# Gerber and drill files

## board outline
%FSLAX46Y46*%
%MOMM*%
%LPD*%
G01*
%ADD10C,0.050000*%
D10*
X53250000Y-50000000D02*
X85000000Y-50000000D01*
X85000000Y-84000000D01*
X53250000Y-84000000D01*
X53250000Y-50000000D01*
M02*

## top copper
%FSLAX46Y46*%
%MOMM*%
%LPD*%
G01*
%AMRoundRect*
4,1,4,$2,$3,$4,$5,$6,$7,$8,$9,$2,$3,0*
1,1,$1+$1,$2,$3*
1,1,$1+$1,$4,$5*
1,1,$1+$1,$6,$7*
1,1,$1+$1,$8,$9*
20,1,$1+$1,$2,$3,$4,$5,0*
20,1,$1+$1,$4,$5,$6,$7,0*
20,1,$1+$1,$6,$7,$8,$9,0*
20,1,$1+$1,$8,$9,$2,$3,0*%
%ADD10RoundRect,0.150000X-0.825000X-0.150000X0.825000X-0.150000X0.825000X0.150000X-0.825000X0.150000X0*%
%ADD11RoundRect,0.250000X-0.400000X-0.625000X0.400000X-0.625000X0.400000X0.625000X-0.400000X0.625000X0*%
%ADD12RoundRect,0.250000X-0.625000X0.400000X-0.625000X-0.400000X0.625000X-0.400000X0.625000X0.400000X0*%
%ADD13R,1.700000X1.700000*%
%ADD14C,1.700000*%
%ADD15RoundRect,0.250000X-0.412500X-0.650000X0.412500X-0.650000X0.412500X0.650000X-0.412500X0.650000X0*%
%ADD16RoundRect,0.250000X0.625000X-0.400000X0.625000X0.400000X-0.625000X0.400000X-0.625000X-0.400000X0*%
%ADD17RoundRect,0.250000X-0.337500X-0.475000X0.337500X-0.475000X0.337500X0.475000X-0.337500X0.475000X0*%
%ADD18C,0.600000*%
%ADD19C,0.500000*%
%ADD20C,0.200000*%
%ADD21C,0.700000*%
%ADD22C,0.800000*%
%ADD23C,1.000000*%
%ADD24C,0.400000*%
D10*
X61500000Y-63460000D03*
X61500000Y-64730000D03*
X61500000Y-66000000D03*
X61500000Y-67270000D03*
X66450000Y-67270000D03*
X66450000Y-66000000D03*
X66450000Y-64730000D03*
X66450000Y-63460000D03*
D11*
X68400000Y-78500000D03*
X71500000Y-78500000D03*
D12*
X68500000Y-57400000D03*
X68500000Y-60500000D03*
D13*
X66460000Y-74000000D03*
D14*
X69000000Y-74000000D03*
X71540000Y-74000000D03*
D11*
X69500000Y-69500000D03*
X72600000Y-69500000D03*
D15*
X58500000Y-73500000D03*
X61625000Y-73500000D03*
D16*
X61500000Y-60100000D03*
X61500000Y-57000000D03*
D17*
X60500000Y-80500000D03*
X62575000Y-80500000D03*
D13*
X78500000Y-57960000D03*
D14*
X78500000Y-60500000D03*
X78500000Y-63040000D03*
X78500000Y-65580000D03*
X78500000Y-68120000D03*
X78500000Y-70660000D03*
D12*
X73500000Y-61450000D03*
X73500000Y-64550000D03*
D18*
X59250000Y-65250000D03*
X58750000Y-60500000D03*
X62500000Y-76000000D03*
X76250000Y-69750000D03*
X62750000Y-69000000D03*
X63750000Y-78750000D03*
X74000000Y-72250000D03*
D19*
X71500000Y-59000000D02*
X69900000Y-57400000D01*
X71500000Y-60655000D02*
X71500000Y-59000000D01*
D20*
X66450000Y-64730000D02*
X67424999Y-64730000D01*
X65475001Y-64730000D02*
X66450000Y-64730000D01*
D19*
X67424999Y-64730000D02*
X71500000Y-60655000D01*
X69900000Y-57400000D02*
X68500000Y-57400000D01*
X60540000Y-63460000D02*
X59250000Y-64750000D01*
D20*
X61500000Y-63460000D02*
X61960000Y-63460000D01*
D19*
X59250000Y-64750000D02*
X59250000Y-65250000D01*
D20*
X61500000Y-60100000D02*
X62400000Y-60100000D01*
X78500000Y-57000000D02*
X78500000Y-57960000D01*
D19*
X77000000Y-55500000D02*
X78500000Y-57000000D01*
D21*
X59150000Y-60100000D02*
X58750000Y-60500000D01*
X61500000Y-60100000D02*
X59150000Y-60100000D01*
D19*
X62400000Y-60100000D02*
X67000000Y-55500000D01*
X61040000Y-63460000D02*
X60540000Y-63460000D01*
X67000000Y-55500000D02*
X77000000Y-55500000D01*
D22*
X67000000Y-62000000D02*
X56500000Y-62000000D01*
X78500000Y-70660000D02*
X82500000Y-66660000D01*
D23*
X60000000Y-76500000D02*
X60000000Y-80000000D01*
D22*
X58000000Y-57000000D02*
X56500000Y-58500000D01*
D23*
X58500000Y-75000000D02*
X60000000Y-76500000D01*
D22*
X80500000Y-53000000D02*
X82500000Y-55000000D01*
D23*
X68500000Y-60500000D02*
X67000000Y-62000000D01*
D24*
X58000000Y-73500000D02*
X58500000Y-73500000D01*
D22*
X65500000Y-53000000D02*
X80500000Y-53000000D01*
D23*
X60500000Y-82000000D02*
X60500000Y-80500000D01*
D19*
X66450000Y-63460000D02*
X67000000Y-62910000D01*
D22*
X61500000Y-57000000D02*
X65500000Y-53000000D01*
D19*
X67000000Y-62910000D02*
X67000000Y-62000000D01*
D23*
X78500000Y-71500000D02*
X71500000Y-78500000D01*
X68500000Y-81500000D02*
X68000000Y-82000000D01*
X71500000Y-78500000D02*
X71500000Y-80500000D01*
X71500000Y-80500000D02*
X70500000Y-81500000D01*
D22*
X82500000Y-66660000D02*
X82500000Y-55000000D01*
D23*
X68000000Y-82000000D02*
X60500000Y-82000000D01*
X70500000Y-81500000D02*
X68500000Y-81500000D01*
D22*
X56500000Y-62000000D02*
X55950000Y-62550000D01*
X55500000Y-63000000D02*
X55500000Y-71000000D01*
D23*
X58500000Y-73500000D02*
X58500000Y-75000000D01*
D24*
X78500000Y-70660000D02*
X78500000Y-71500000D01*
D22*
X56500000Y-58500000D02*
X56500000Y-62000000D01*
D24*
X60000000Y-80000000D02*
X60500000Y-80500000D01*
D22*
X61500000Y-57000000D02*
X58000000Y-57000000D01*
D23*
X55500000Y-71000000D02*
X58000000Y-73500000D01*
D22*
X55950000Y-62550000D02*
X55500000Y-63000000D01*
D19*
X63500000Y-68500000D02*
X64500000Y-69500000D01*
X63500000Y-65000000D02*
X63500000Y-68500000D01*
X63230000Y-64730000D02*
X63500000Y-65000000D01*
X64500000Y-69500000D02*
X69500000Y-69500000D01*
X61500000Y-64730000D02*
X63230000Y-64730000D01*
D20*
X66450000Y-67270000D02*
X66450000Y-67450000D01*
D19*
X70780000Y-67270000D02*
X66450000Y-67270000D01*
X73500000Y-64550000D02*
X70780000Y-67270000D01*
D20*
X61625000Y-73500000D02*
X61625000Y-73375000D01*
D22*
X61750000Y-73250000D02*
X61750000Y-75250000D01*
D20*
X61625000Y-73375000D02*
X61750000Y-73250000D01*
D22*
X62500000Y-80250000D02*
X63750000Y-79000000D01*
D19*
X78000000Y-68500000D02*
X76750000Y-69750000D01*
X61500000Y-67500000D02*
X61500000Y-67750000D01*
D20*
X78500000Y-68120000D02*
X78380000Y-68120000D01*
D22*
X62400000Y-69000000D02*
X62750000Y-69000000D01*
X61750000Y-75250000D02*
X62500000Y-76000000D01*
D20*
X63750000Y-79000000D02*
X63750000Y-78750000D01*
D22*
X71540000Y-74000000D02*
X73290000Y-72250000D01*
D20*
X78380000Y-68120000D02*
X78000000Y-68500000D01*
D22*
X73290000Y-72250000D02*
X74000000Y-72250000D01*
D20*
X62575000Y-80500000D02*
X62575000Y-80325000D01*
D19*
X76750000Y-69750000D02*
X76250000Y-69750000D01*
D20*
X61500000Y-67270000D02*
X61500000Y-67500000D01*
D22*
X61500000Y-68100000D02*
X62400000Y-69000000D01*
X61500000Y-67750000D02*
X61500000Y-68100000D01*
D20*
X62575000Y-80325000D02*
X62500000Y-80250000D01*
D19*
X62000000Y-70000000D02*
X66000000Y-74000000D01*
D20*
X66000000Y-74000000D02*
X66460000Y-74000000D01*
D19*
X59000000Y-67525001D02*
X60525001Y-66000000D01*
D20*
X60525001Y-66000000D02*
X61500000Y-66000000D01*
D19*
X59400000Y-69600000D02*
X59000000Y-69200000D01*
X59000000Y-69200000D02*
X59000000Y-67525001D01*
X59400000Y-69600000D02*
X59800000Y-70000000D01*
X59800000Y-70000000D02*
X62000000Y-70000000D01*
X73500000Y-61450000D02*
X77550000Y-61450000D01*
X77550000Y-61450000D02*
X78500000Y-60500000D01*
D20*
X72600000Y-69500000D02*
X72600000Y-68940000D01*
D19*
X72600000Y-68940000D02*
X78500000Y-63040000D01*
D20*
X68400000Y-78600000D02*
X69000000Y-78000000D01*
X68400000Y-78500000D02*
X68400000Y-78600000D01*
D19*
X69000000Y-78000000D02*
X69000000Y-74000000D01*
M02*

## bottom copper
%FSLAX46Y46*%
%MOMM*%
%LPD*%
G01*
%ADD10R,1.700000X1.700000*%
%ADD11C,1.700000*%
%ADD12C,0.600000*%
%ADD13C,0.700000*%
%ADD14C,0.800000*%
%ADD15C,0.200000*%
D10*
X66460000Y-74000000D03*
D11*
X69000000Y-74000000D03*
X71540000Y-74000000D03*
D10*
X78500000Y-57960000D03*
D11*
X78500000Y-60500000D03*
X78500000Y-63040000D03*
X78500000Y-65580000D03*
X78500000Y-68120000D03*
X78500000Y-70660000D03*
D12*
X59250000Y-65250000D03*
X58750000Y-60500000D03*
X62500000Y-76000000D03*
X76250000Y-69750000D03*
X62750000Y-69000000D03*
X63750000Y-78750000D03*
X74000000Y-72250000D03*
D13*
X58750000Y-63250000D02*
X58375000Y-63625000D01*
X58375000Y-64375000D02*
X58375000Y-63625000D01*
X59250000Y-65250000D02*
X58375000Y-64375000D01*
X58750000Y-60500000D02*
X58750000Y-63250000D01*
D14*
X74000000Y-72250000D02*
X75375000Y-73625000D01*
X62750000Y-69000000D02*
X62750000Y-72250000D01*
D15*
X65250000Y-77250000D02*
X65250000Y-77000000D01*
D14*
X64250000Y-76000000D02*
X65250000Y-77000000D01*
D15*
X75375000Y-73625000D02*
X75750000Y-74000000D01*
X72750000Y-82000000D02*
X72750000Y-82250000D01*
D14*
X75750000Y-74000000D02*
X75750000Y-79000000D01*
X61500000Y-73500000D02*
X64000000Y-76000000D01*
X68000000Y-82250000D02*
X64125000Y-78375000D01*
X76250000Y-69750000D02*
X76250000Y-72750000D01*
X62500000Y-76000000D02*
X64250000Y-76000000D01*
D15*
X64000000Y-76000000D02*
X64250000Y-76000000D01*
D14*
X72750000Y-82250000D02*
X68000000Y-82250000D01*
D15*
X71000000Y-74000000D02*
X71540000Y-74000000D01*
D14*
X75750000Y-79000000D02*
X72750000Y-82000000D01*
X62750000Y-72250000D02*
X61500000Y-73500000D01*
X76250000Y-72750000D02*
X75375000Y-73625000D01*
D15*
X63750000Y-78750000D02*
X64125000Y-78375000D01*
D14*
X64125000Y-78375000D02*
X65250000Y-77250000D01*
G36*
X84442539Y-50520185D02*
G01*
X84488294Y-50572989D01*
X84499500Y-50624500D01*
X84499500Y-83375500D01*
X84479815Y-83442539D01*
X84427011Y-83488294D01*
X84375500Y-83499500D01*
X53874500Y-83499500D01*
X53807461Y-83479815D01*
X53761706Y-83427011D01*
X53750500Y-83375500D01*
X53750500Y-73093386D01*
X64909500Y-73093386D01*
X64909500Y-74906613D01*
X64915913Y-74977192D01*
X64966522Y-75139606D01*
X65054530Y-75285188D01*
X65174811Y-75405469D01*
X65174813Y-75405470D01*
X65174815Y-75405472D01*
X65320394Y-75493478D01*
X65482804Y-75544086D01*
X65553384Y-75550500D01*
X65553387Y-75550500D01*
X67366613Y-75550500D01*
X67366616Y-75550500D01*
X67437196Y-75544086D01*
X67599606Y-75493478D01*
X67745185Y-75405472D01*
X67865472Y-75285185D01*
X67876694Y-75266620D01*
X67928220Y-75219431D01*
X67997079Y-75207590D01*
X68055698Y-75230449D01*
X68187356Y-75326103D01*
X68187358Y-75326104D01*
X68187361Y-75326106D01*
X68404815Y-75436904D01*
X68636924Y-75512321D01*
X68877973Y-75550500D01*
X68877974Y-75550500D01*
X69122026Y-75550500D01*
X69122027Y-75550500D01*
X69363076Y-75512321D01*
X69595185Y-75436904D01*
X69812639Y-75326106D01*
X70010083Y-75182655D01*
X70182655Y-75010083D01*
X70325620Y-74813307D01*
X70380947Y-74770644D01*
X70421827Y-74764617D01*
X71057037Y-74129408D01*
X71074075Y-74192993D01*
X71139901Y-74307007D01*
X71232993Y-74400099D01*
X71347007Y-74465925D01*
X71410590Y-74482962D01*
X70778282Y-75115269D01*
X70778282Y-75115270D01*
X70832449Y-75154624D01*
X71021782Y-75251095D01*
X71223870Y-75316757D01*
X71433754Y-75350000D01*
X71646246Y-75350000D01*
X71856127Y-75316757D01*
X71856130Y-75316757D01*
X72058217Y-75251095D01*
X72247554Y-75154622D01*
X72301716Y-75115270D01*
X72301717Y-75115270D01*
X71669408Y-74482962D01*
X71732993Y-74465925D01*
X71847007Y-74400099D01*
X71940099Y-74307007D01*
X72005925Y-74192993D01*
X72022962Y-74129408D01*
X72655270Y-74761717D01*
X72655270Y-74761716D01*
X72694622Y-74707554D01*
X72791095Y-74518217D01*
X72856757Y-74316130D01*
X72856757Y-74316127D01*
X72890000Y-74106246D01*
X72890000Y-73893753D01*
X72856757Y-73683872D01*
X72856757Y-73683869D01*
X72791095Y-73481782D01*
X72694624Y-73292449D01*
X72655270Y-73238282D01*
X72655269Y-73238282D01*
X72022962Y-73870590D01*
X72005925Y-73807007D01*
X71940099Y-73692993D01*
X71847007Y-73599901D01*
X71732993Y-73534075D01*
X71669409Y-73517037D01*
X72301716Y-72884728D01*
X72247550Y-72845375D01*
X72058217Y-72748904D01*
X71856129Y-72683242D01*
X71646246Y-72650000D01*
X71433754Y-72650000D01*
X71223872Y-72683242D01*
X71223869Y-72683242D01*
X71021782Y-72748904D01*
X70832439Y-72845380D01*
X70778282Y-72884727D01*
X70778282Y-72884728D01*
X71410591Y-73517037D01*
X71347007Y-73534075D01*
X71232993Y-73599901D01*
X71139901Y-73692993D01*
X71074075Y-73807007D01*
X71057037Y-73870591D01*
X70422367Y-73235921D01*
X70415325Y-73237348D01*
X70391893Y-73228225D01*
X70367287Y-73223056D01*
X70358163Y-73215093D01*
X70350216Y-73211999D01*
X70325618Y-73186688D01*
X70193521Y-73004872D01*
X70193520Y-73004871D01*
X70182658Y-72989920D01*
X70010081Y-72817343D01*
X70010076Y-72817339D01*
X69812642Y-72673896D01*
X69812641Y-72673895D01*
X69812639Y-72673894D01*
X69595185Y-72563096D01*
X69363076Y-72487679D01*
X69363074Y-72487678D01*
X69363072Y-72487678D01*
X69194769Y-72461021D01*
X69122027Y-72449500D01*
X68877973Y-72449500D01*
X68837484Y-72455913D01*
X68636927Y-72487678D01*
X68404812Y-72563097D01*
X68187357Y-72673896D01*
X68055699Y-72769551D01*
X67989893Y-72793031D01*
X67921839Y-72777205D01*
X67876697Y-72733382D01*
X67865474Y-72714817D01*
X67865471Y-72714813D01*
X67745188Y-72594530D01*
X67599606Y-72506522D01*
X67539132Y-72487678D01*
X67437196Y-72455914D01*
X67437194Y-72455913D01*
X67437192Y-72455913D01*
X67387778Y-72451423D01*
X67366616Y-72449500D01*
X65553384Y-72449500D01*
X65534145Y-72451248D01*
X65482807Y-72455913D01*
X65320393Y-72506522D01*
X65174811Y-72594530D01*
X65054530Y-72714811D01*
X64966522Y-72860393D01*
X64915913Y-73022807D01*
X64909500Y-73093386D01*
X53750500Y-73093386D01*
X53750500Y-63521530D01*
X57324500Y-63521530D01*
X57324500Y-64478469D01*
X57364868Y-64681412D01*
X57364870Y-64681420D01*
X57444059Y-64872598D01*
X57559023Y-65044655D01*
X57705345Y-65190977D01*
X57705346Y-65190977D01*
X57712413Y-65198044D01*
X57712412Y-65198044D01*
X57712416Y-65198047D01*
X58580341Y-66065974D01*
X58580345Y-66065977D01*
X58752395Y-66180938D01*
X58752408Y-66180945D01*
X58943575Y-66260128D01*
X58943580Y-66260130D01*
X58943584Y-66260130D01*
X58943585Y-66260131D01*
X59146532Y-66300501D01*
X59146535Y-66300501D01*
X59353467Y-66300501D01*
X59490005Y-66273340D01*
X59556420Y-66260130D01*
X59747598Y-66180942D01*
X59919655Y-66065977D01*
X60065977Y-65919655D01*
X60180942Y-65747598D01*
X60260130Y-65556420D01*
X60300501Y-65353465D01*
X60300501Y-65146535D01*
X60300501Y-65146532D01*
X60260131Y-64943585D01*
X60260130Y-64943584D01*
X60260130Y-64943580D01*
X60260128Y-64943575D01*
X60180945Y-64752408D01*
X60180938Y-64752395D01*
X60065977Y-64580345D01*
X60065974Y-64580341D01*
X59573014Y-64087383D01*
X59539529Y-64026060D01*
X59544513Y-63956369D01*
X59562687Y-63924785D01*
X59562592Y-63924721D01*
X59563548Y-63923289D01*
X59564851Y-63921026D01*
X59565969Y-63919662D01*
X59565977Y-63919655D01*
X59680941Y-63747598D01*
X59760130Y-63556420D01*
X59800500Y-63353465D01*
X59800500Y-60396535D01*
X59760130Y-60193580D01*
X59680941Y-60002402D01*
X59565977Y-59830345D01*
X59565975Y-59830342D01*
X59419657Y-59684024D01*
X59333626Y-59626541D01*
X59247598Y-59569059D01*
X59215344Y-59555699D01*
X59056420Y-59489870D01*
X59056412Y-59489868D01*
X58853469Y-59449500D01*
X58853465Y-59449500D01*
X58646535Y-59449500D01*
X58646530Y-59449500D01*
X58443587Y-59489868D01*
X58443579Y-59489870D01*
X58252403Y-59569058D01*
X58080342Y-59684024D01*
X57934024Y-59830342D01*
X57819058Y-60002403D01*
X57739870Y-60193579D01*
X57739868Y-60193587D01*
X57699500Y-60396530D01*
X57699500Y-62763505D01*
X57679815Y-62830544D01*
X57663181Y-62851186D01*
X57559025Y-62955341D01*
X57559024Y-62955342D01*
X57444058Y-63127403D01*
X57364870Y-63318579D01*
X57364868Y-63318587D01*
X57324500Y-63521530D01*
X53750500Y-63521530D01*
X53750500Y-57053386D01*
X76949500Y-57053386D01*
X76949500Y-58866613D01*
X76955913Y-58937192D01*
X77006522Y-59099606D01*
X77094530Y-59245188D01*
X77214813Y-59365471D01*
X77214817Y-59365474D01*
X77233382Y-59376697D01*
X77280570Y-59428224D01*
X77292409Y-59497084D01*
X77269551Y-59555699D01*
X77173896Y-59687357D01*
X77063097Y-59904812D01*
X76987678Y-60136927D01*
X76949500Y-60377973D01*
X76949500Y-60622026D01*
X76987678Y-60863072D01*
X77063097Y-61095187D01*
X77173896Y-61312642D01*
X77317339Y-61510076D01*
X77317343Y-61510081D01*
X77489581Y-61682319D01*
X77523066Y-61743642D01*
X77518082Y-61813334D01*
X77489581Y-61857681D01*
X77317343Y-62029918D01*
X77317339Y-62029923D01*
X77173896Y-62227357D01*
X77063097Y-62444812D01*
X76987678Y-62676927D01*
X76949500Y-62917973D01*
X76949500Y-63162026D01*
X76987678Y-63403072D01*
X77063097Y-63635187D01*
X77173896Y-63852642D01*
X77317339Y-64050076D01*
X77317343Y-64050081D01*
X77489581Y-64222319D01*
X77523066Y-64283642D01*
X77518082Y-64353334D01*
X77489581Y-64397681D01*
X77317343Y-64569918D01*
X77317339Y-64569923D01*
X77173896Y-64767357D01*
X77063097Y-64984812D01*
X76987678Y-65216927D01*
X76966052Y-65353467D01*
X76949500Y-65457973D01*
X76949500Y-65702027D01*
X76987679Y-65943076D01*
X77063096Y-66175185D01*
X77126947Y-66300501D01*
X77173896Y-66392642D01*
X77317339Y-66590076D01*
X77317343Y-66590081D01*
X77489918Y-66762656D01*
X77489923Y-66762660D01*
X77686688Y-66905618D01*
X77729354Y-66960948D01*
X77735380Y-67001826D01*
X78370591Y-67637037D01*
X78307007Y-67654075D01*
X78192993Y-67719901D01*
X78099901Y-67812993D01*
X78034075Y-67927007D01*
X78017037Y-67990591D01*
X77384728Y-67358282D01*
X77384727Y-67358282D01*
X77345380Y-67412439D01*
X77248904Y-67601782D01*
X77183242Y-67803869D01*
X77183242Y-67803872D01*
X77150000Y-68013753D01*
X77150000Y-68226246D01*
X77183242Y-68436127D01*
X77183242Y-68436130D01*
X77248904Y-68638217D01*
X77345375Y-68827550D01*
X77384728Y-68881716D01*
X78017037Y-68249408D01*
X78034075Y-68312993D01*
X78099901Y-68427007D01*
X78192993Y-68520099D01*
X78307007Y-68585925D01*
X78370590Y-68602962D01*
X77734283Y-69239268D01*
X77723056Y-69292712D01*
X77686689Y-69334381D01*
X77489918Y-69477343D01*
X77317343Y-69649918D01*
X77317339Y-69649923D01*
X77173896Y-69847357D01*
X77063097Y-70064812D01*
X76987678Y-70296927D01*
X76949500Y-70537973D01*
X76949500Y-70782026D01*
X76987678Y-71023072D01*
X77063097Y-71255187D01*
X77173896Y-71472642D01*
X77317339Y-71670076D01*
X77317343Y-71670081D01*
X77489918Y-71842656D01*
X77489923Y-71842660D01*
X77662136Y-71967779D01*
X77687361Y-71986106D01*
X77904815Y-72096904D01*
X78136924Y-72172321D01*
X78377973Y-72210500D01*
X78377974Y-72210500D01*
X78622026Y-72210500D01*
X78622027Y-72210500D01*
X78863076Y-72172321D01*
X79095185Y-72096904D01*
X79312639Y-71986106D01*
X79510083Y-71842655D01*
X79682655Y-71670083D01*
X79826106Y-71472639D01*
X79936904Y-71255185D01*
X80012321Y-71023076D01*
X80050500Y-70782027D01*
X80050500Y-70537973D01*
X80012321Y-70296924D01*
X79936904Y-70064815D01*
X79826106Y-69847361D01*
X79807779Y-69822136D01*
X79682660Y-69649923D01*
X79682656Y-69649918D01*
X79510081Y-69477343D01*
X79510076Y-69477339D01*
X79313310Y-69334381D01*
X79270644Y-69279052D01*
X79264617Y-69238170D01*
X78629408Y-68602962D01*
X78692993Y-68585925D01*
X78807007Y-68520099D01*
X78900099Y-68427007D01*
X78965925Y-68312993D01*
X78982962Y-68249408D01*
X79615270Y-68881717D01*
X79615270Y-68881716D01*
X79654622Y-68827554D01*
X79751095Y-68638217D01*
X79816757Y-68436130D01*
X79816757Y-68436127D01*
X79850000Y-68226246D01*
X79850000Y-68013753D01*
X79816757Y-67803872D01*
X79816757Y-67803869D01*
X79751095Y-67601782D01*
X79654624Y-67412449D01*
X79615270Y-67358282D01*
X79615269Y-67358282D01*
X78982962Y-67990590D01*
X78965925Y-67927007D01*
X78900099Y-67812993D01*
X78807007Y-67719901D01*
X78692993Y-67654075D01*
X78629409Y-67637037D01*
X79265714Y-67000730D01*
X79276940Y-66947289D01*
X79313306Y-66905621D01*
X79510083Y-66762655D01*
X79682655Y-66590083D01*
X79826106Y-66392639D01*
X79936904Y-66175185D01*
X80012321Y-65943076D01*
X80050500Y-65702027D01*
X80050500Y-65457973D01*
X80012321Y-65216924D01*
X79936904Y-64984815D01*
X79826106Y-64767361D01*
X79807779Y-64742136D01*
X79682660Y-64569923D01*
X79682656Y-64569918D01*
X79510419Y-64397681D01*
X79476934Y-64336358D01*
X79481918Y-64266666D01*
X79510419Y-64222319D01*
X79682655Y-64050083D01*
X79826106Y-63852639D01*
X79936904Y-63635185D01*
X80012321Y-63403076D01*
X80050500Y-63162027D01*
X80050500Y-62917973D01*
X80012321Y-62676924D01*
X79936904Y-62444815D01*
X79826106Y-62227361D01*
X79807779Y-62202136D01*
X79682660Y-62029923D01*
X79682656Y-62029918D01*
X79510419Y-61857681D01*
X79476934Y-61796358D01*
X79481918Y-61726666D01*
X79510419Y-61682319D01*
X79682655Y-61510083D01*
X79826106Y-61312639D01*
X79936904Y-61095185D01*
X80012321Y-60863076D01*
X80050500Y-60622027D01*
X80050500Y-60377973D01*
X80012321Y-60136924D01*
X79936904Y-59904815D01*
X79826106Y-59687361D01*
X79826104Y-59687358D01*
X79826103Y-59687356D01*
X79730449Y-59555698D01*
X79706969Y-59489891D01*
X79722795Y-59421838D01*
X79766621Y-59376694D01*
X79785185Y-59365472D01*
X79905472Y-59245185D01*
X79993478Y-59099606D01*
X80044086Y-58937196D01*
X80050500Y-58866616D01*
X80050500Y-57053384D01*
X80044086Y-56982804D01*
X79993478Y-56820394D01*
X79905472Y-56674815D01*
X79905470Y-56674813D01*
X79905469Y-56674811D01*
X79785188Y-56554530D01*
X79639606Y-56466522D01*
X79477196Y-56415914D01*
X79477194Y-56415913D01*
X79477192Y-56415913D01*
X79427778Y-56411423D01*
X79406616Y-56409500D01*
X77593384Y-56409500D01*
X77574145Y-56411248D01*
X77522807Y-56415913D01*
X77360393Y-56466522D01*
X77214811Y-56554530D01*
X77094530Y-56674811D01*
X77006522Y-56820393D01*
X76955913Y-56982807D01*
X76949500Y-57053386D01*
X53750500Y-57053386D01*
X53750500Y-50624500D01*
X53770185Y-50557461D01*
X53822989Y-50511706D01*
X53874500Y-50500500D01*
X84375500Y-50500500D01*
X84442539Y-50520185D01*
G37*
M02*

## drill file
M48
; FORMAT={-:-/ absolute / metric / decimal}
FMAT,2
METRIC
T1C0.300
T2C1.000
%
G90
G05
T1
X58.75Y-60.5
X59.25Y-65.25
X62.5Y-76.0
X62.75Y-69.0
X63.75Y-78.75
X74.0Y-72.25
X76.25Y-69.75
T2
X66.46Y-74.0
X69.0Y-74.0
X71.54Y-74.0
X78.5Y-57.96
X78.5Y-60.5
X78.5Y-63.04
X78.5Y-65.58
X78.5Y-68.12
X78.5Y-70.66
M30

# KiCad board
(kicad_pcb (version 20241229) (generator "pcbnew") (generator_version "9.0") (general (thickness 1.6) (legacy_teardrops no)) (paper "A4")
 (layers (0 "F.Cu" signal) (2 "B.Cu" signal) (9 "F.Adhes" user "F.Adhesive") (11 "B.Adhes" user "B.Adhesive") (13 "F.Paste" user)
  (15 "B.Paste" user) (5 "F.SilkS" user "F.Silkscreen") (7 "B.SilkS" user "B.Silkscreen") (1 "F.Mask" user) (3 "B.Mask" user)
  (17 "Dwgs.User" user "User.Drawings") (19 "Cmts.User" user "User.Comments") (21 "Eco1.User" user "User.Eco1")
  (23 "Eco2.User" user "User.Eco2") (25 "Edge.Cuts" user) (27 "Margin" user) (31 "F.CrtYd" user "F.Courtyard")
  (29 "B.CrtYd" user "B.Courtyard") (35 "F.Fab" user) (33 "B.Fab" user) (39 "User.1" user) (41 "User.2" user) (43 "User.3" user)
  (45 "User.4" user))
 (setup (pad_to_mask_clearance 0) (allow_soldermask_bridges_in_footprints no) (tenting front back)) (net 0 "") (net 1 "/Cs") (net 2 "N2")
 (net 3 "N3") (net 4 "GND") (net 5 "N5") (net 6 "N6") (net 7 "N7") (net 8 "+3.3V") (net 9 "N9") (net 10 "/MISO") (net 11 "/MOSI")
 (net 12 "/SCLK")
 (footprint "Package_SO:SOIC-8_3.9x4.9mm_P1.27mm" (layer "F.Cu") (at 63.975 65.365)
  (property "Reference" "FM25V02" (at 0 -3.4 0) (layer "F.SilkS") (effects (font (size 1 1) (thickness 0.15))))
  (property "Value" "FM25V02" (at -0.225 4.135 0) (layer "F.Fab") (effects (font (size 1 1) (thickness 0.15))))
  (pad "1" smd roundrect (at -2.475 -1.905) (size 1.95 0.6) (layers "F.Cu" "F.Mask" "F.Paste") (roundrect_rratio 0.25) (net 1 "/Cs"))
  (pad "2" smd roundrect (at -2.475 -0.635) (size 1.95 0.6) (layers "F.Cu" "F.Mask" "F.Paste") (roundrect_rratio 0.25) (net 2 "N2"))
  (pad "3" smd roundrect (at -2.475 0.635) (size 1.95 0.6) (layers "F.Cu" "F.Mask" "F.Paste") (roundrect_rratio 0.25) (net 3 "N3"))
  (pad "4" smd roundrect (at -2.475 1.905) (size 1.95 0.6) (layers "F.Cu" "F.Mask" "F.Paste") (roundrect_rratio 0.25) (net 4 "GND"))
  (pad "5" smd roundrect (at 2.475 1.905) (size 1.95 0.6) (layers "F.Cu" "F.Mask" "F.Paste") (roundrect_rratio 0.25) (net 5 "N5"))
  (pad "6" smd roundrect (at 2.475 0.635) (size 1.95 0.6) (layers "F.Cu" "F.Mask" "F.Paste") (roundrect_rratio 0.25) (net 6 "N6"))
  (pad "7" smd roundrect (at 2.475 -0.635) (size 1.95 0.6) (layers "F.Cu" "F.Mask" "F.Paste") (roundrect_rratio 0.25) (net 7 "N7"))
  (pad "8" smd roundrect (at 2.475 -1.905) (size 1.95 0.6) (layers "F.Cu" "F.Mask" "F.Paste") (roundrect_rratio 0.25) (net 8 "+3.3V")))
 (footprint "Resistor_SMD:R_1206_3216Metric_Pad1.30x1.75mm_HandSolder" (layer "F.Cu") (at 69.95 78.5)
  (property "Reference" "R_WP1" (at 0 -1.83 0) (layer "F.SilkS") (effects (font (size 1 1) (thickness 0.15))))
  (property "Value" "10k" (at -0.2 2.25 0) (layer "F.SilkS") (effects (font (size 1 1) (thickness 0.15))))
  (pad "1" smd roundrect (at -1.55 0) (size 1.3 1.75) (layers "F.Cu" "F.Mask" "F.Paste") (roundrect_rratio 0.192308) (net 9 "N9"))
  (pad "2" smd roundrect (at 1.55 0) (size 1.3 1.75) (layers "F.Cu" "F.Mask" "F.Paste") (roundrect_rratio 0.192308) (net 8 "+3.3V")))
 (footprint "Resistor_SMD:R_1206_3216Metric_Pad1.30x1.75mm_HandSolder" (layer "F.Cu") (at 68.5 58.95 -90)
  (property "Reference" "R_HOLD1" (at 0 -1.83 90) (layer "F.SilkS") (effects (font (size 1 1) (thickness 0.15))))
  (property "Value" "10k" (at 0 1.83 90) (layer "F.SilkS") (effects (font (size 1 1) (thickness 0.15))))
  (pad "1" smd roundrect (at -1.55 0 270) (size 1.3 1.75) (layers "F.Cu" "F.Mask" "F.Paste") (roundrect_rratio 0.192308) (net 7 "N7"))
  (pad "2" smd roundrect (at 1.55 0 270) (size 1.3 1.75) (layers "F.Cu" "F.Mask" "F.Paste") (roundrect_rratio 0.192308) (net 8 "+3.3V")))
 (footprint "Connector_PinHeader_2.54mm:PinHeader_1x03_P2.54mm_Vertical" (layer "F.Cu") (at 66.46 74 90)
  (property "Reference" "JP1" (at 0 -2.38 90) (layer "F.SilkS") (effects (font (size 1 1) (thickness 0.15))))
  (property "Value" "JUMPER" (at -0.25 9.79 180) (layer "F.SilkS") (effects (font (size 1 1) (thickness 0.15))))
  (pad "1" thru_hole rect (at 0 0 90) (size 1.7 1.7) (drill 1) (layers "*.Cu" "*.Mask") (remove_unused_layers no) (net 3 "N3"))
  (pad "2" thru_hole circle (at 0 2.54 90) (size 1.7 1.7) (drill 1) (layers "*.Cu" "*.Mask") (remove_unused_layers no) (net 9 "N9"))
  (pad "3" thru_hole circle (at 0 5.08 90) (size 1.7 1.7) (drill 1) (layers "*.Cu" "*.Mask") (remove_unused_layers no) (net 4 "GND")))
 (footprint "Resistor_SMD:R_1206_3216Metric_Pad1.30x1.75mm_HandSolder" (layer "F.Cu") (at 71.05 69.5)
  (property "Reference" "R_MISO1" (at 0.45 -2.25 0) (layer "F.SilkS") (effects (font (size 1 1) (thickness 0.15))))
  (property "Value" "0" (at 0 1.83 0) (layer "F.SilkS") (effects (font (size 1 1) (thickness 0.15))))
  (pad "1" smd roundrect (at -1.55 0) (size 1.3 1.75) (layers "F.Cu" "F.Mask" "F.Paste") (roundrect_rratio 0.192308) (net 2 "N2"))
  (pad "2" smd roundrect (at 1.55 0) (size 1.3 1.75) (layers "F.Cu" "F.Mask" "F.Paste") (roundrect_rratio 0.192308) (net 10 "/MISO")))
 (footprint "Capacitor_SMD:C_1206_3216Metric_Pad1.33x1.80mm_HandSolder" (layer "F.Cu") (at 60.0625 73.5)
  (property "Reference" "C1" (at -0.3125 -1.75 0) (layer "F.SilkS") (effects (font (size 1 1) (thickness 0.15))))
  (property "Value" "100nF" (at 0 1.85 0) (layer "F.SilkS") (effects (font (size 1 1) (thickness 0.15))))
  (pad "1" smd roundrect (at -1.5625 0) (size 1.325 1.8) (layers "F.Cu" "F.Mask" "F.Paste") (roundrect_rratio 0.188679) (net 8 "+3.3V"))
  (pad "2" smd roundrect (at 1.5625 0) (size 1.325 1.8) (layers "F.Cu" "F.Mask" "F.Paste") (roundrect_rratio 0.188679) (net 4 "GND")))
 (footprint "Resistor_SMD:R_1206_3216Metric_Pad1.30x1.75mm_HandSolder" (layer "F.Cu") (at 61.5 58.55 90)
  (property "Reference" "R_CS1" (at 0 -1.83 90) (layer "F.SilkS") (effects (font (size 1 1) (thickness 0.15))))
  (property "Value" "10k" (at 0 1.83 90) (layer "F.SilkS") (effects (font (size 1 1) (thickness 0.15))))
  (pad "1" smd roundrect (at -1.55 0 90) (size 1.3 1.75) (layers "F.Cu" "F.Mask" "F.Paste") (roundrect_rratio 0.192308) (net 1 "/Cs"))
  (pad "2" smd roundrect (at 1.55 0 90) (size 1.3 1.75) (layers "F.Cu" "F.Mask" "F.Paste") (roundrect_rratio 0.192308) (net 8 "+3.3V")))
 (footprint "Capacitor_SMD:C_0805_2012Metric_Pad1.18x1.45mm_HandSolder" (layer "F.Cu") (at 61.5375 80.5)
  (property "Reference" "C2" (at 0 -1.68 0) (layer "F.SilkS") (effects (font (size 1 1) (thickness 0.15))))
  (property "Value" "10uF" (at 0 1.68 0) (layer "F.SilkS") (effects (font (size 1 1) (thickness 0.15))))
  (pad "1" smd roundrect (at -1.0375 0) (size 1.175 1.45) (layers "F.Cu" "F.Mask" "F.Paste") (roundrect_rratio 0.212766) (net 8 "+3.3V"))
  (pad "2" smd roundrect (at 1.0375 0) (size 1.175 1.45) (layers "F.Cu" "F.Mask" "F.Paste") (roundrect_rratio 0.212766) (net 4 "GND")))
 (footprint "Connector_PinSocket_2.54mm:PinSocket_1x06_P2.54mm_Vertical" (layer "F.Cu") (at 78.5 57.96)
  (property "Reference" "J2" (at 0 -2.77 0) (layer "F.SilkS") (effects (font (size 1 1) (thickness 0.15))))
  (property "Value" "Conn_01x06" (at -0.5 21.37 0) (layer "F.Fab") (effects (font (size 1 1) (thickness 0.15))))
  (pad "1" thru_hole rect (at 0 0) (size 1.7 1.7) (drill 1) (layers "*.Cu" "*.Mask") (remove_unused_layers no) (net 1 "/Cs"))
  (pad "2" thru_hole circle (at 0 2.54) (size 1.7 1.7) (drill 1) (layers "*.Cu" "*.Mask") (remove_unused_layers no) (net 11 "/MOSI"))
  (pad "3" thru_hole circle (at 0 5.08) (size 1.7 1.7) (drill 1) (layers "*.Cu" "*.Mask") (remove_unused_layers no) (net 10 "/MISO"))
  (pad "4" thru_hole circle (at 0 7.62) (size 1.7 1.7) (drill 1) (layers "*.Cu" "*.Mask") (remove_unused_layers no) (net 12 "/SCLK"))
  (pad "5" thru_hole circle (at 0 10.16) (size 1.7 1.7) (drill 1) (layers "*.Cu" "*.Mask") (remove_unused_layers no) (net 4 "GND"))
  (pad "6" thru_hole circle (at 0 12.7) (size 1.7 1.7) (drill 1) (layers "*.Cu" "*.Mask") (remove_unused_layers no) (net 8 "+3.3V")))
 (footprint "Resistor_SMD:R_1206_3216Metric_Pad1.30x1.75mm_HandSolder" (layer "F.Cu") (at 73.5 63 -90)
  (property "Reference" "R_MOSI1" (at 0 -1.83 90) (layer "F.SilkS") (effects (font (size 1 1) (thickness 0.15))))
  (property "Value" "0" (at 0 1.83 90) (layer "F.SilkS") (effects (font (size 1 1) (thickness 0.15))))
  (pad "1" smd roundrect (at -1.55 0 270) (size 1.3 1.75) (layers "F.Cu" "F.Mask" "F.Paste") (roundrect_rratio 0.192308) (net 11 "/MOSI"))
  (pad "2" smd roundrect (at 1.55 0 270) (size 1.3 1.75) (layers "F.Cu" "F.Mask" "F.Paste") (roundrect_rratio 0.192308) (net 5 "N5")))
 (gr_rect (start 53.25 50) (end 85 84) (stroke (width 0.05) (type default)) (fill no) (layer "Edge.Cuts"))
 (segment (start 71.5 59) (end 69.9 57.4) (width 0.5) (layer "F.Cu") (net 7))
 (segment (start 71.5 60.655) (end 71.5 59) (width 0.5) (layer "F.Cu") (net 7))
 (segment (start 66.45 64.73) (end 67.424999 64.73) (width 0.2) (layer "F.Cu") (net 7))
 (segment (start 65.475001 64.73) (end 66.45 64.73) (width 0.2) (layer "F.Cu") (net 7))
 (segment (start 67.424999 64.73) (end 71.5 60.655) (width 0.5) (layer "F.Cu") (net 7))
 (segment (start 69.9 57.4) (end 68.5 57.4) (width 0.5) (layer "F.Cu") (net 7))
 (segment (start 60.54 63.46) (end 59.25 64.75) (width 0.5) (layer "F.Cu") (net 1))
 (segment (start 61.5 63.46) (end 61.96 63.46) (width 0.2) (layer "F.Cu") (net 1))
 (segment (start 59.25 64.75) (end 59.25 65.25) (width 0.5) (layer "F.Cu") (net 1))
 (segment (start 61.5 60.1) (end 62.4 60.1) (width 0.2) (layer "F.Cu") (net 1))
 (segment (start 78.5 57) (end 78.5 57.96) (width 0.2) (layer "F.Cu") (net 1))
 (segment (start 77 55.5) (end 78.5 57) (width 0.5) (layer "F.Cu") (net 1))
 (segment (start 59.15 60.1) (end 58.75 60.5) (width 0.7) (layer "F.Cu") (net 1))
 (segment (start 61.5 60.1) (end 59.15 60.1) (width 0.7) (layer "F.Cu") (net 1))
 (segment (start 62.4 60.1) (end 67 55.5) (width 0.5) (layer "F.Cu") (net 1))
 (segment (start 61.04 63.46) (end 60.54 63.46) (width 0.5) (layer "F.Cu") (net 1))
 (segment (start 67 55.5) (end 77 55.5) (width 0.5) (layer "F.Cu") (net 1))
 (via (at 59.25 65.25) (size 0.6) (drill 0.3) (layers "F.Cu" "B.Cu") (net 1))
 (via (at 58.75 60.5) (size 0.6) (drill 0.3) (layers "F.Cu" "B.Cu") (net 1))
 (segment (start 58.75 63.25) (end 58.375 63.625) (width 0.7) (layer "B.Cu") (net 1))
 (segment (start 58.375 64.375) (end 58.375 63.625) (width 0.7) (layer "B.Cu") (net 1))
 (segment (start 59.25 65.25) (end 58.375 64.375) (width 0.7) (layer "B.Cu") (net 1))
 (segment (start 58.75 60.5) (end 58.75 63.25) (width 0.7) (layer "B.Cu") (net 1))
 (segment (start 67 62) (end 56.5 62) (width 0.8) (layer "F.Cu") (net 8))
 (segment (start 78.5 70.66) (end 82.5 66.66) (width 0.8) (layer "F.Cu") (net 8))
 (segment (start 60 76.5) (end 60 80) (width 1) (layer "F.Cu") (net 8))
 (segment (start 58 57) (end 56.5 58.5) (width 0.8) (layer "F.Cu") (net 8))
 (segment (start 58.5 75) (end 60 76.5) (width 1) (layer "F.Cu") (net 8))
 (segment (start 80.5 53) (end 82.5 55) (width 0.8) (layer "F.Cu") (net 8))
 (segment (start 68.5 60.5) (end 67 62) (width 1) (layer "F.Cu") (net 8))
 (segment (start 58 73.5) (end 58.5 73.5) (width 0.4) (layer "F.Cu") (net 8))
 (segment (start 65.5 53) (end 80.5 53) (width 0.8) (layer "F.Cu") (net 8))
 (segment (start 60.5 82) (end 60.5 80.5) (width 1) (layer "F.Cu") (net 8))
 (segment (start 66.45 63.46) (end 67 62.91) (width 0.5) (layer "F.Cu") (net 8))
 (segment (start 61.5 57) (end 65.5 53) (width 0.8) (layer "F.Cu") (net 8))
 (segment (start 67 62.91) (end 67 62) (width 0.5) (layer "F.Cu") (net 8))
 (segment (start 78.5 71.5) (end 71.5 78.5) (width 1) (layer "F.Cu") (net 8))
 (segment (start 68.5 81.5) (end 68 82) (width 1) (layer "F.Cu") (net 8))
 (segment (start 71.5 78.5) (end 71.5 80.5) (width 1) (layer "F.Cu") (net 8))
 (segment (start 71.5 80.5) (end 70.5 81.5) (width 1) (layer "F.Cu") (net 8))
 (segment (start 82.5 66.66) (end 82.5 55) (width 0.8) (layer "F.Cu") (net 8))
 (segment (start 68 82) (end 60.5 82) (width 1) (layer "F.Cu") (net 8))
 (segment (start 70.5 81.5) (end 68.5 81.5) (width 1) (layer "F.Cu") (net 8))
 (segment (start 56.5 62) (end 55.95 62.55) (width 0.8) (layer "F.Cu") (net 8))
 (segment (start 55.5 63) (end 55.5 71) (width 0.8) (layer "F.Cu") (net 8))
 (segment (start 58.5 73.5) (end 58.5 75) (width 1) (layer "F.Cu") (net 8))
 (segment (start 78.5 70.66) (end 78.5 71.5) (width 0.4) (layer "F.Cu") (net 8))
 (segment (start 56.5 58.5) (end 56.5 62) (width 0.8) (layer "F.Cu") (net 8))
 (segment (start 60 80) (end 60.5 80.5) (width 0.4) (layer "F.Cu") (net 8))
 (segment (start 61.5 57) (end 58 57) (width 0.8) (layer "F.Cu") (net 8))
 (segment (start 55.5 71) (end 58 73.5) (width 1) (layer "F.Cu") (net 8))
 (segment (start 55.95 62.55) (end 55.5 63) (width 0.8) (layer "F.Cu") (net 8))
 (segment (start 63.5 68.5) (end 64.5 69.5) (width 0.5) (layer "F.Cu") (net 2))
 (segment (start 63.5 65) (end 63.5 68.5) (width 0.5) (layer "F.Cu") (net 2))
 (segment (start 63.23 64.73) (end 63.5 65) (width 0.5) (layer "F.Cu") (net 2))
 (segment (start 64.5 69.5) (end 69.5 69.5) (width 0.5) (layer "F.Cu") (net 2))
 (segment (start 61.5 64.73) (end 63.23 64.73) (width 0.5) (layer "F.Cu") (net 2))
 (segment (start 66.45 67.27) (end 66.45 67.45) (width 0.2) (layer "F.Cu") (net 5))
 (segment (start 70.78 67.27) (end 66.45 67.27) (width 0.5) (layer "F.Cu") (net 5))
 (segment (start 73.5 64.55) (end 70.78 67.27) (width 0.5) (layer "F.Cu") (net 5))
 (segment (start 61.625 73.5) (end 61.625 73.375) (width 0.2) (layer "F.Cu") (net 4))
 (segment (start 61.75 73.25) (end 61.75 75.25) (width 0.8) (layer "F.Cu") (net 4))
 (segment (start 61.625 73.375) (end 61.75 73.25) (width 0.2) (layer "F.Cu") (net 4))
 (segment (start 62.5 80.25) (end 63.75 79) (width 0.8) (layer "F.Cu") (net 4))
 (segment (start 78 68.5) (end 76.75 69.75) (width 0.5) (layer "F.Cu") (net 4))
 (segment (start 61.5 67.5) (end 61.5 67.75) (width 0.5) (layer "F.Cu") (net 4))
 (segment (start 78.5 68.12) (end 78.38 68.12) (width 0.2) (layer "F.Cu") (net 4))
 (segment (start 62.4 69) (end 62.75 69) (width 0.8) (layer "F.Cu") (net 4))
 (segment (start 61.75 75.25) (end 62.5 76) (width 0.8) (layer "F.Cu") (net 4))
 (segment (start 63.75 79) (end 63.75 78.75) (width 0.2) (layer "F.Cu") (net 4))
 (segment (start 71.54 74) (end 73.29 72.25) (width 0.8) (layer "F.Cu") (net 4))
 (segment (start 78.38 68.12) (end 78 68.5) (width 0.2) (layer "F.Cu") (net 4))
 (segment (start 73.29 72.25) (end 74 72.25) (width 0.8) (layer "F.Cu") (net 4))
 (segment (start 62.575 80.5) (end 62.575 80.325) (width 0.2) (layer "F.Cu") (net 4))
 (segment (start 76.75 69.75) (end 76.25 69.75) (width 0.5) (layer "F.Cu") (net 4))
 (segment (start 61.5 67.27) (end 61.5 67.5) (width 0.2) (layer "F.Cu") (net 4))
 (segment (start 61.5 68.1) (end 62.4 69) (width 0.8) (layer "F.Cu") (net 4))
 (segment (start 61.5 67.75) (end 61.5 68.1) (width 0.8) (layer "F.Cu") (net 4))
 (segment (start 62.575 80.325) (end 62.5 80.25) (width 0.2) (layer "F.Cu") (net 4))
 (via (at 62.5 76) (size 0.6) (drill 0.3) (layers "F.Cu" "B.Cu") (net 4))
 (via (at 76.25 69.75) (size 0.6) (drill 0.3) (layers "F.Cu" "B.Cu") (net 4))
 (via (at 62.75 69) (size 0.6) (drill 0.3) (layers "F.Cu" "B.Cu") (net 4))
 (via (at 63.75 78.75) (size 0.6) (drill 0.3) (layers "F.Cu" "B.Cu") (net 4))
 (via (at 74 72.25) (size 0.6) (drill 0.3) (layers "F.Cu" "B.Cu") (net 4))
 (segment (start 74 72.25) (end 75.375 73.625) (width 0.8) (layer "B.Cu") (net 4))
 (segment (start 62.75 69) (end 62.75 72.25) (width 0.8) (layer "B.Cu") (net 4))
 (segment (start 65.25 77.25) (end 65.25 77) (width 0.2) (layer "B.Cu") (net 4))
 (segment (start 64.25 76) (end 65.25 77) (width 0.8) (layer "B.Cu") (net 4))
 (segment (start 75.375 73.625) (end 75.75 74) (width 0.2) (layer "B.Cu") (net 4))
 (segment (start 72.75 82) (end 72.75 82.25) (width 0.2) (layer "B.Cu") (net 4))
 (segment (start 75.75 74) (end 75.75 79) (width 0.8) (layer "B.Cu") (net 4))
 (segment (start 61.5 73.5) (end 64 76) (width 0.8) (layer "B.Cu") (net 4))
 (segment (start 68 82.25) (end 64.125 78.375) (width 0.8) (layer "B.Cu") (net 4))
 (segment (start 76.25 69.75) (end 76.25 72.75) (width 0.8) (layer "B.Cu") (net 4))
 (segment (start 62.5 76) (end 64.25 76) (width 0.8) (layer "B.Cu") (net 4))
 (segment (start 64 76) (end 64.25 76) (width 0.2) (layer "B.Cu") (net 4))
 (segment (start 72.75 82.25) (end 68 82.25) (width 0.8) (layer "B.Cu") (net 4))
 (segment (start 71 74) (end 71.54 74) (width 0.2) (layer "B.Cu") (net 4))
 (segment (start 75.75 79) (end 72.75 82) (width 0.8) (layer "B.Cu") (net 4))
 (segment (start 62.75 72.25) (end 61.5 73.5) (width 0.8) (layer "B.Cu") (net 4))
 (segment (start 76.25 72.75) (end 75.375 73.625) (width 0.8) (layer "B.Cu") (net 4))
 (segment (start 63.75 78.75) (end 64.125 78.375) (width 0.2) (layer "B.Cu") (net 4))
 (segment (start 64.125 78.375) (end 65.25 77.25) (width 0.8) (layer "B.Cu") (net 4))
 (segment (start 62 70) (end 66 74) (width 0.5) (layer "F.Cu") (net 3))
 (segment (start 66 74) (end 66.46 74) (width 0.2) (layer "F.Cu") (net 3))
 (segment (start 59 67.525001) (end 60.525001 66) (width 0.5) (layer "F.Cu") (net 3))
 (segment (start 60.525001 66) (end 61.5 66) (width 0.2) (layer "F.Cu") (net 3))
 (segment (start 59.4 69.6) (end 59 69.2) (width 0.5) (layer "F.Cu") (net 3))
 (segment (start 59 69.2) (end 59 67.525001) (width 0.5) (layer "F.Cu") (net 3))
 (segment (start 59.4 69.6) (end 59.8 70) (width 0.5) (layer "F.Cu") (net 3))
 (segment (start 59.8 70) (end 62 70) (width 0.5) (layer "F.Cu") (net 3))
 (segment (start 73.5 61.45) (end 77.55 61.45) (width 0.5) (layer "F.Cu") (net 11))
 (segment (start 77.55 61.45) (end 78.5 60.5) (width 0.5) (layer "F.Cu") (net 11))
 (segment (start 72.6 69.5) (end 72.6 68.94) (width 0.2) (layer "F.Cu") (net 10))
 (segment (start 72.6 68.94) (end 78.5 63.04) (width 0.5) (layer "F.Cu") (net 10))
 (segment (start 68.4 78.6) (end 69 78) (width 0.2) (layer "F.Cu") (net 9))
 (segment (start 68.4 78.5) (end 68.4 78.6) (width 0.2) (layer "F.Cu") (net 9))
 (segment (start 69 78) (end 69 74) (width 0.5) (layer "F.Cu") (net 9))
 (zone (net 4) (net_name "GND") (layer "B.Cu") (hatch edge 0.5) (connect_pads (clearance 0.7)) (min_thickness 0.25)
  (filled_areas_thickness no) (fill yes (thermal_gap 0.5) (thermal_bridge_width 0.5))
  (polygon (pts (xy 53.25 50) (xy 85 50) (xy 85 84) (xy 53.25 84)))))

